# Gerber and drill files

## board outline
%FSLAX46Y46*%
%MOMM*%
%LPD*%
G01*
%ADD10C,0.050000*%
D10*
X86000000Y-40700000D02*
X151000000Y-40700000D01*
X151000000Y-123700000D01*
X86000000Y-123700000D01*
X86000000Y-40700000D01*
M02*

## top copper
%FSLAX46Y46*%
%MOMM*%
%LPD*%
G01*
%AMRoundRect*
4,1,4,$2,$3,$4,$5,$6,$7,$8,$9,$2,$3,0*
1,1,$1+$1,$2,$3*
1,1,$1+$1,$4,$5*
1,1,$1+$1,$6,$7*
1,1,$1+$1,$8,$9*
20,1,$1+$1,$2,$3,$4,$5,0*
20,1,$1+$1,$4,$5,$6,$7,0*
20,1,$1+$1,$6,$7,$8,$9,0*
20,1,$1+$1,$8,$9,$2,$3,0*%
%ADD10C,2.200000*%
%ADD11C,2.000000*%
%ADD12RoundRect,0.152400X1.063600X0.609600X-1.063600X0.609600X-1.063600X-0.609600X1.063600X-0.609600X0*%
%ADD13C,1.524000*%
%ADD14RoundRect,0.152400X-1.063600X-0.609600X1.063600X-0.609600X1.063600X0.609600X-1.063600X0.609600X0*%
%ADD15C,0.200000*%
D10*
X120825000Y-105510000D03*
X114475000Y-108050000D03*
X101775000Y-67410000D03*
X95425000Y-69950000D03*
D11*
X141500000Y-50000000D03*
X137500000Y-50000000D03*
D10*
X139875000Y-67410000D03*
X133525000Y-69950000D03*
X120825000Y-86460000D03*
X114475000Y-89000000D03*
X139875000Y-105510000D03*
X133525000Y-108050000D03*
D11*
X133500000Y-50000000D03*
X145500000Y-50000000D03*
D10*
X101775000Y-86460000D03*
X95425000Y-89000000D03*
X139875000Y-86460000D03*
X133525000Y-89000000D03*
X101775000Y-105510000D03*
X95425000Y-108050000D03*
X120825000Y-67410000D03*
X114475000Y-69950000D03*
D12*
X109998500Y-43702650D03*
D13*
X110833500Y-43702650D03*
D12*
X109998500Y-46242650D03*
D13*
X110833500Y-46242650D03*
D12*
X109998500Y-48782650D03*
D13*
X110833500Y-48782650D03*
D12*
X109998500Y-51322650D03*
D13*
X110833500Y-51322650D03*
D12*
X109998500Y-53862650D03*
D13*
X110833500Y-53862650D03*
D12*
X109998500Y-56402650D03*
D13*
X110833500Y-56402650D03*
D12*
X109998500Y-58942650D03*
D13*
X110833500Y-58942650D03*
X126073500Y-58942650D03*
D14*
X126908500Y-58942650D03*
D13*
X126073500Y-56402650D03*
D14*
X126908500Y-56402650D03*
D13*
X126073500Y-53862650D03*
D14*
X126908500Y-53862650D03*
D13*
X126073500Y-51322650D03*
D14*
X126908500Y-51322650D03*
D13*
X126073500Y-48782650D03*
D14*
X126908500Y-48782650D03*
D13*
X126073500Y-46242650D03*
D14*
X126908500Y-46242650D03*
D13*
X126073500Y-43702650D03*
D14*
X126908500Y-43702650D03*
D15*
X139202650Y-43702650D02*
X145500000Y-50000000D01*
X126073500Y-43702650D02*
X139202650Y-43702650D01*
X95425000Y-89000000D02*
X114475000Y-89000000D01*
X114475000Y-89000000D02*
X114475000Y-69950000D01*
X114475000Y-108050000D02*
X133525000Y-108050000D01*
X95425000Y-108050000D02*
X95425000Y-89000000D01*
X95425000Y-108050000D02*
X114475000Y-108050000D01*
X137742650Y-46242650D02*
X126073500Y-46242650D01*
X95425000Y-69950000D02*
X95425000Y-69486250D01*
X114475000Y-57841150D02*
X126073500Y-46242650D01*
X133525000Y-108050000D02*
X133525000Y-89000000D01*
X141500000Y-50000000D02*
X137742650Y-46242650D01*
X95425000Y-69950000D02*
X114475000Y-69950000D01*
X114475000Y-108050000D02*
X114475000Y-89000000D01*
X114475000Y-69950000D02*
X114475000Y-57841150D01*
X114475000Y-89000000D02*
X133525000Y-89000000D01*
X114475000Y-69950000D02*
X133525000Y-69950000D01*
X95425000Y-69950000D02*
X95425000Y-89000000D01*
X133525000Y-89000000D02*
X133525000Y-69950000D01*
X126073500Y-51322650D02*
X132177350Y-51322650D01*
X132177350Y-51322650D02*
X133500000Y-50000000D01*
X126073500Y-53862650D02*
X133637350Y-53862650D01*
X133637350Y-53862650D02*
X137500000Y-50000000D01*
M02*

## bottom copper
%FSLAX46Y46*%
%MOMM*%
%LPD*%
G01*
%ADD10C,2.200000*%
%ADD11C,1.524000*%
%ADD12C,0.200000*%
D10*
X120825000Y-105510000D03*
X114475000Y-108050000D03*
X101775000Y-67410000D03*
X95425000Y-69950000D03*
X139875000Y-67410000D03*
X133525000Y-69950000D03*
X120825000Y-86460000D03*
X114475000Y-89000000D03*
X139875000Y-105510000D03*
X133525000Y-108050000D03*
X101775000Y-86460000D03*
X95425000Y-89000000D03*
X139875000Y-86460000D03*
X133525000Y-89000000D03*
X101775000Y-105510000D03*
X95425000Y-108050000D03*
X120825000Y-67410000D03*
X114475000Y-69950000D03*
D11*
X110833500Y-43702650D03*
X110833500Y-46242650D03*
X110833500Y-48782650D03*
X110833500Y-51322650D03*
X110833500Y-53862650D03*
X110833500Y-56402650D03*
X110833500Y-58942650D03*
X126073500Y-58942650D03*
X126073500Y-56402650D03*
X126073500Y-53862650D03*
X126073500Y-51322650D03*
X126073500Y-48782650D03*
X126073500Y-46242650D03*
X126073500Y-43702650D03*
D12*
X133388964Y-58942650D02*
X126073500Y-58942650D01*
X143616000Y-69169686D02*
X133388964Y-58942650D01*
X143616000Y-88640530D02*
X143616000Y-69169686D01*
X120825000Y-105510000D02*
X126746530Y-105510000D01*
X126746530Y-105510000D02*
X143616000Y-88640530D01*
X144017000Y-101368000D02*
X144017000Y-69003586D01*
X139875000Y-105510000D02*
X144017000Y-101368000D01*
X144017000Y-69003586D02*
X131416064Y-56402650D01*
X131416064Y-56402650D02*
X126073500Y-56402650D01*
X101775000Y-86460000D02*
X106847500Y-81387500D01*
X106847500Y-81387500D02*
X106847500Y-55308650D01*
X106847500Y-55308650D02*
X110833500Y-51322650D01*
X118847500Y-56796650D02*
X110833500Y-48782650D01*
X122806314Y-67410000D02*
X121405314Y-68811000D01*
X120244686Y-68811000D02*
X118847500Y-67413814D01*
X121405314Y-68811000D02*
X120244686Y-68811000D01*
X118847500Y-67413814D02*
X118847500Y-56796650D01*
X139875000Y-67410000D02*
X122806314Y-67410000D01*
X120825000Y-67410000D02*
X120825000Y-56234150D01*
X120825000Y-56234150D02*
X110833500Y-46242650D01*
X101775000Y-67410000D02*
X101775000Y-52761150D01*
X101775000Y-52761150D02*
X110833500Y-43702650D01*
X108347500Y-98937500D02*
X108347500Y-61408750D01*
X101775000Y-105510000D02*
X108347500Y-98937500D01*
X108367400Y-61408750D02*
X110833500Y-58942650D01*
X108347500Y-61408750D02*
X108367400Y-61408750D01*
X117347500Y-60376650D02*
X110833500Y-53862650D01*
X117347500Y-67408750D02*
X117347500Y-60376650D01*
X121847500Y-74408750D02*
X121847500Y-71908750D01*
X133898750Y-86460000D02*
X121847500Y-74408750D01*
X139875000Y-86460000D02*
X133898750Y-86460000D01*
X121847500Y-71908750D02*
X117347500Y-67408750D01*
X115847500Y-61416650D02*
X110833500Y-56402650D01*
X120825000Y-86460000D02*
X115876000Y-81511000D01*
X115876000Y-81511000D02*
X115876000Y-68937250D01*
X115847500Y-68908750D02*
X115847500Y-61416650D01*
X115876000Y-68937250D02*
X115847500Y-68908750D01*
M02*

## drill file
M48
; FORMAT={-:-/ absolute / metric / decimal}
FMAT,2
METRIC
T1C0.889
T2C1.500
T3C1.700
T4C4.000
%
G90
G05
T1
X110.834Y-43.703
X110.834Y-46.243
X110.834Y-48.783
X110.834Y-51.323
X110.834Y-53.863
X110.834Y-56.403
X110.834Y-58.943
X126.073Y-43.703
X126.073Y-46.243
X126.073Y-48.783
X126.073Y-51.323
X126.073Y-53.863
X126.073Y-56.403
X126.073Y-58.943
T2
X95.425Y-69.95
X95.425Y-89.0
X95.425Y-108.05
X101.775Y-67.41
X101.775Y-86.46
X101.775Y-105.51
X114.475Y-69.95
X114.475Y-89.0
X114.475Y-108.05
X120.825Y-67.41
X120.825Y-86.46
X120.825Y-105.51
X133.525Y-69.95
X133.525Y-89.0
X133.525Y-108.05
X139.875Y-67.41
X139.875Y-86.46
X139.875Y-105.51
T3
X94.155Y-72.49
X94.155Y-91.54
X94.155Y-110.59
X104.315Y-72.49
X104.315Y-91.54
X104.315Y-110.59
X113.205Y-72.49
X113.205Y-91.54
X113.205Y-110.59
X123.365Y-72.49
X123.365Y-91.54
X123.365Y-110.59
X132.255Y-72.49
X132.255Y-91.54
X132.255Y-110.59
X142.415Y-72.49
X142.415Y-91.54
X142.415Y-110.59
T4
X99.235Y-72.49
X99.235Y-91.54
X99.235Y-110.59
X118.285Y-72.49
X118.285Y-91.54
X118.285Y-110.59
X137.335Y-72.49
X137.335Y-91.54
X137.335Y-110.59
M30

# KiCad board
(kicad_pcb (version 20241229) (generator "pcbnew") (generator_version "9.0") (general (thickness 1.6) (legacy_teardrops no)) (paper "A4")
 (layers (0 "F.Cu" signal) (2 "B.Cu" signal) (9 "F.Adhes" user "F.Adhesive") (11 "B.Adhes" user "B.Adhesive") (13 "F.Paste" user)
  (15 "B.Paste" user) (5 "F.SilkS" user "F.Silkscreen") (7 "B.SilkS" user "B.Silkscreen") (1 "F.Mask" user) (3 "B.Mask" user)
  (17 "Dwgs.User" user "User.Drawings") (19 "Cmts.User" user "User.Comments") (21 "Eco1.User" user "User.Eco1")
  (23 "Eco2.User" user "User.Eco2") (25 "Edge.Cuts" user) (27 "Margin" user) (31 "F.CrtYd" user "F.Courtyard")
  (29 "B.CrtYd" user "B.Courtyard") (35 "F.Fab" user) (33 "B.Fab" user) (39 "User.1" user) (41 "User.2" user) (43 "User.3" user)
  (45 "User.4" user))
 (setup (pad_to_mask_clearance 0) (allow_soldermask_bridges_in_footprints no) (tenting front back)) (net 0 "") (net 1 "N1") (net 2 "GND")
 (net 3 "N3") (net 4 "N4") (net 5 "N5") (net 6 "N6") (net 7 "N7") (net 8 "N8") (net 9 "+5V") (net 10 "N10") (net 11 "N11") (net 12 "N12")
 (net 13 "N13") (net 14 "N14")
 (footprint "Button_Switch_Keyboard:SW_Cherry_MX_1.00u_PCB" (layer "F.Cu") (at 120.825 105.51)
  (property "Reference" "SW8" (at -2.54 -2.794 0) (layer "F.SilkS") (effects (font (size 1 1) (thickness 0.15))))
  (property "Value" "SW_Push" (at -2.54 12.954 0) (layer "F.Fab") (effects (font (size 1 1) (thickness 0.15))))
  (pad "" np_thru_hole circle (at -7.62 5.08) (size 1.7 1.7) (drill 1.7) (layers "*.Cu" "*.Mask"))
  (pad "" np_thru_hole circle (at -2.54 5.08) (size 4 4) (drill 4) (layers "*.Cu" "*.Mask"))
  (pad "" np_thru_hole circle (at 2.54 5.08) (size 1.7 1.7) (drill 1.7) (layers "*.Cu" "*.Mask"))
  (pad "1" thru_hole circle (at 0 0) (size 2.2 2.2) (drill 1.5) (layers "*.Cu" "*.Mask") (remove_unused_layers no) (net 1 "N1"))
  (pad "2" thru_hole circle (at -6.35 2.54) (size 2.2 2.2) (drill 1.5) (layers "*.Cu" "*.Mask") (remove_unused_layers no) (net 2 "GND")))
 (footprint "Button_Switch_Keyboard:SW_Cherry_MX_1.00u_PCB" (layer "F.Cu") (at 101.775 67.41)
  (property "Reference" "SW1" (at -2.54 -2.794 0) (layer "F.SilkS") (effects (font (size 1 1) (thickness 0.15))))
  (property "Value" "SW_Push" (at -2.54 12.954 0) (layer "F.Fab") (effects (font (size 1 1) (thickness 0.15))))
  (pad "" np_thru_hole circle (at -7.62 5.08) (size 1.7 1.7) (drill 1.7) (layers "*.Cu" "*.Mask"))
  (pad "" np_thru_hole circle (at -2.54 5.08) (size 4 4) (drill 4) (layers "*.Cu" "*.Mask"))
  (pad "" np_thru_hole circle (at 2.54 5.08) (size 1.7 1.7) (drill 1.7) (layers "*.Cu" "*.Mask"))
  (pad "1" thru_hole circle (at 0 0) (size 2.2 2.2) (drill 1.5) (layers "*.Cu" "*.Mask") (remove_unused_layers no) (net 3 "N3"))
  (pad "2" thru_hole circle (at -6.35 2.54) (size 2.2 2.2) (drill 1.5) (layers "*.Cu" "*.Mask") (remove_unused_layers no) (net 2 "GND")))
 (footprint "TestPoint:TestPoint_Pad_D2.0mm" (layer "F.Cu") (at 141.5 50)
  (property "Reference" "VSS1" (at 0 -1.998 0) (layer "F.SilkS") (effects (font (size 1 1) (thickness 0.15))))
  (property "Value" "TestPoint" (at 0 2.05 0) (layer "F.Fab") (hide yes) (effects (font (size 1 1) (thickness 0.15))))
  (pad "1" smd circle (at 0 0) (size 2 2) (layers "F.Cu" "F.Mask") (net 2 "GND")))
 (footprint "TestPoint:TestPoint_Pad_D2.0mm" (layer "F.Cu") (at 137.5 50)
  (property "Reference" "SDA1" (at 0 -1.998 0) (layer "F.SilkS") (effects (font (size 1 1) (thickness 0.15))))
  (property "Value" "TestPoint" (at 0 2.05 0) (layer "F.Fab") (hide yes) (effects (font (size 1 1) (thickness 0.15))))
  (pad "1" smd circle (at 0 0) (size 2 2) (layers "F.Cu" "F.Mask") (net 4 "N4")))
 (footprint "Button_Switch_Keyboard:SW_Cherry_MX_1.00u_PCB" (layer "F.Cu") (at 139.875 67.41)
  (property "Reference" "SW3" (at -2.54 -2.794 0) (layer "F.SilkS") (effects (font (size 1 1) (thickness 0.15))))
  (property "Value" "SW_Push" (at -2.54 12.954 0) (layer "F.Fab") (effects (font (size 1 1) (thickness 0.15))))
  (pad "" np_thru_hole circle (at -7.62 5.08) (size 1.7 1.7) (drill 1.7) (layers "*.Cu" "*.Mask"))
  (pad "" np_thru_hole circle (at -2.54 5.08) (size 4 4) (drill 4) (layers "*.Cu" "*.Mask"))
  (pad "" np_thru_hole circle (at 2.54 5.08) (size 1.7 1.7) (drill 1.7) (layers "*.Cu" "*.Mask"))
  (pad "1" thru_hole circle (at 0 0) (size 2.2 2.2) (drill 1.5) (layers "*.Cu" "*.Mask") (remove_unused_layers no) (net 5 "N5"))
  (pad "2" thru_hole circle (at -6.35 2.54) (size 2.2 2.2) (drill 1.5) (layers "*.Cu" "*.Mask") (remove_unused_layers no) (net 2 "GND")))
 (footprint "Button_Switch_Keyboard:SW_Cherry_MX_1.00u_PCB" (layer "F.Cu") (at 120.825 86.46)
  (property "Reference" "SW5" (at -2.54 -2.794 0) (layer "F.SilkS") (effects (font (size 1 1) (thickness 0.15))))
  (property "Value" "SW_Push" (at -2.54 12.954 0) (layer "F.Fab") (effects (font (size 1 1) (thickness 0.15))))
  (pad "" np_thru_hole circle (at -7.62 5.08) (size 1.7 1.7) (drill 1.7) (layers "*.Cu" "*.Mask"))
  (pad "" np_thru_hole circle (at -2.54 5.08) (size 4 4) (drill 4) (layers "*.Cu" "*.Mask"))
  (pad "" np_thru_hole circle (at 2.54 5.08) (size 1.7 1.7) (drill 1.7) (layers "*.Cu" "*.Mask"))
  (pad "1" thru_hole circle (at 0 0) (size 2.2 2.2) (drill 1.5) (layers "*.Cu" "*.Mask") (remove_unused_layers no) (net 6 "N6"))
  (pad "2" thru_hole circle (at -6.35 2.54) (size 2.2 2.2) (drill 1.5) (layers "*.Cu" "*.Mask") (remove_unused_layers no) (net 2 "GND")))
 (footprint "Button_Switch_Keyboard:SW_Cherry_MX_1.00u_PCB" (layer "F.Cu") (at 139.875 105.51)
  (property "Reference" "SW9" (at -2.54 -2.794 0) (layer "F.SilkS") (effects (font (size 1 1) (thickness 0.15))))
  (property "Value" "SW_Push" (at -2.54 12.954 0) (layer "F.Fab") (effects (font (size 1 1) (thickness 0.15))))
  (pad "" np_thru_hole circle (at -7.62 5.08) (size 1.7 1.7) (drill 1.7) (layers "*.Cu" "*.Mask"))
  (pad "" np_thru_hole circle (at -2.54 5.08) (size 4 4) (drill 4) (layers "*.Cu" "*.Mask"))
  (pad "" np_thru_hole circle (at 2.54 5.08) (size 1.7 1.7) (drill 1.7) (layers "*.Cu" "*.Mask"))
  (pad "1" thru_hole circle (at 0 0) (size 2.2 2.2) (drill 1.5) (layers "*.Cu" "*.Mask") (remove_unused_layers no) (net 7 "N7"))
  (pad "2" thru_hole circle (at -6.35 2.54) (size 2.2 2.2) (drill 1.5) (layers "*.Cu" "*.Mask") (remove_unused_layers no) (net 2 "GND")))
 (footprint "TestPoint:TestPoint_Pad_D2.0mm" (layer "F.Cu") (at 133.5 50)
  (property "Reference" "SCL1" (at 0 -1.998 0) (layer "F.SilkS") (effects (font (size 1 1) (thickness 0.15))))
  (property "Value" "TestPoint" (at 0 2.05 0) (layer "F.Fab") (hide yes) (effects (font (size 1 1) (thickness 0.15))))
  (pad "1" smd circle (at 0 0) (size 2 2) (layers "F.Cu" "F.Mask") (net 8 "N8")))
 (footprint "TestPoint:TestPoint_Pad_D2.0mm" (layer "F.Cu") (at 145.5 50)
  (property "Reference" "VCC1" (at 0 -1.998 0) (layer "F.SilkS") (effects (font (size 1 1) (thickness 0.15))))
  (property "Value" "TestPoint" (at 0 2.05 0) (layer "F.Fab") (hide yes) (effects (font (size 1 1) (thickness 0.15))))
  (pad "1" smd circle (at 0 0) (size 2 2) (layers "F.Cu" "F.Mask") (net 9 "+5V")))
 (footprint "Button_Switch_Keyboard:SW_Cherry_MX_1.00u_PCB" (layer "F.Cu") (at 101.775 86.46)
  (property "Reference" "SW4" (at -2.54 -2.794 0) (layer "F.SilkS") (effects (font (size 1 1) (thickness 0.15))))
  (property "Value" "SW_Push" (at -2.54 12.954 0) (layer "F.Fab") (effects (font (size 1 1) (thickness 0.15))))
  (pad "" np_thru_hole circle (at -7.62 5.08) (size 1.7 1.7) (drill 1.7) (layers "*.Cu" "*.Mask"))
  (pad "" np_thru_hole circle (at -2.54 5.08) (size 4 4) (drill 4) (layers "*.Cu" "*.Mask"))
  (pad "" np_thru_hole circle (at 2.54 5.08) (size 1.7 1.7) (drill 1.7) (layers "*.Cu" "*.Mask"))
  (pad "1" thru_hole circle (at 0 0) (size 2.2 2.2) (drill 1.5) (layers "*.Cu" "*.Mask") (remove_unused_layers no) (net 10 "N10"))
  (pad "2" thru_hole circle (at -6.35 2.54) (size 2.2 2.2) (drill 1.5) (layers "*.Cu" "*.Mask") (remove_unused_layers no) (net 2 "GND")))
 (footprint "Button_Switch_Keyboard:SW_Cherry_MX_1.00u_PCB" (layer "F.Cu") (at 139.875 86.46)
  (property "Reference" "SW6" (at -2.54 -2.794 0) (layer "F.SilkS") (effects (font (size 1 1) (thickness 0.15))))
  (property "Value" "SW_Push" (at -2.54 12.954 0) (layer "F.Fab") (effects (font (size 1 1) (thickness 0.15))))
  (pad "" np_thru_hole circle (at -7.62 5.08) (size 1.7 1.7) (drill 1.7) (layers "*.Cu" "*.Mask"))
  (pad "" np_thru_hole circle (at -2.54 5.08) (size 4 4) (drill 4) (layers "*.Cu" "*.Mask"))
  (pad "" np_thru_hole circle (at 2.54 5.08) (size 1.7 1.7) (drill 1.7) (layers "*.Cu" "*.Mask"))
  (pad "1" thru_hole circle (at 0 0) (size 2.2 2.2) (drill 1.5) (layers "*.Cu" "*.Mask") (remove_unused_layers no) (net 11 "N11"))
  (pad "2" thru_hole circle (at -6.35 2.54) (size 2.2 2.2) (drill 1.5) (layers "*.Cu" "*.Mask") (remove_unused_layers no) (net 2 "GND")))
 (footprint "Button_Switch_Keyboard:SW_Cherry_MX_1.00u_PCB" (layer "F.Cu") (at 101.775 105.51)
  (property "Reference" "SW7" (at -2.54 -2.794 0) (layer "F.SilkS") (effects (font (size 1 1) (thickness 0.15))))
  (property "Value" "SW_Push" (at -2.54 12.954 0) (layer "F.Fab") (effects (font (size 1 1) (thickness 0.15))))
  (pad "" np_thru_hole circle (at -7.62 5.08) (size 1.7 1.7) (drill 1.7) (layers "*.Cu" "*.Mask"))
  (pad "" np_thru_hole circle (at -2.54 5.08) (size 4 4) (drill 4) (layers "*.Cu" "*.Mask"))
  (pad "" np_thru_hole circle (at 2.54 5.08) (size 1.7 1.7) (drill 1.7) (layers "*.Cu" "*.Mask"))
  (pad "1" thru_hole circle (at 0 0) (size 2.2 2.2) (drill 1.5) (layers "*.Cu" "*.Mask") (remove_unused_layers no) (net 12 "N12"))
  (pad "2" thru_hole circle (at -6.35 2.54) (size 2.2 2.2) (drill 1.5) (layers "*.Cu" "*.Mask") (remove_unused_layers no) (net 2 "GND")))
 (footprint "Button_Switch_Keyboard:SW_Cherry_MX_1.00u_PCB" (layer "F.Cu") (at 120.825 67.41)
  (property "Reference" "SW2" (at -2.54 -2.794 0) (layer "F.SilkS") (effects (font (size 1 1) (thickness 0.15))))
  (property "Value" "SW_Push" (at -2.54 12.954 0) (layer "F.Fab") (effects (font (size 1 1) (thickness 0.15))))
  (pad "" np_thru_hole circle (at -7.62 5.08) (size 1.7 1.7) (drill 1.7) (layers "*.Cu" "*.Mask"))
  (pad "" np_thru_hole circle (at -2.54 5.08) (size 4 4) (drill 4) (layers "*.Cu" "*.Mask"))
  (pad "" np_thru_hole circle (at 2.54 5.08) (size 1.7 1.7) (drill 1.7) (layers "*.Cu" "*.Mask"))
  (pad "1" thru_hole circle (at 0 0) (size 2.2 2.2) (drill 1.5) (layers "*.Cu" "*.Mask") (remove_unused_layers no) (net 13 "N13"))
  (pad "2" thru_hole circle (at -6.35 2.54) (size 2.2 2.2) (drill 1.5) (layers "*.Cu" "*.Mask") (remove_unused_layers no) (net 2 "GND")))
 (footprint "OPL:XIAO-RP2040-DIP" (layer "F.Cu") (at 118.4535 51.32265)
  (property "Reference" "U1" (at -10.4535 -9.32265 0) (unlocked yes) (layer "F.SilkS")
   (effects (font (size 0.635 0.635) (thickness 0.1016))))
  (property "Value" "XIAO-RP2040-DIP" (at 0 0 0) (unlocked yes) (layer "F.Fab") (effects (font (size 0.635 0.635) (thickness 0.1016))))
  (pad "1" smd roundrect (at -8.455 -7.62 180) (size 2.432 1.524) (layers "F.Cu" "F.Mask") (roundrect_rratio 0.1) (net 3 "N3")
   (thermal_bridge_angle 45))
  (pad "1" thru_hole circle (at -7.62 -7.62 180) (size 1.524 1.524) (drill 0.889) (layers "*.Cu" "*.Mask") (remove_unused_layers no)
   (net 3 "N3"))
  (pad "2" smd roundrect (at -8.455 -5.08 180) (size 2.432 1.524) (layers "F.Cu" "F.Mask") (roundrect_rratio 0.1) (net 13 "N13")
   (thermal_bridge_angle 45))
  (pad "2" thru_hole circle (at -7.62 -5.08 180) (size 1.524 1.524) (drill 0.889) (layers "*.Cu" "*.Mask") (remove_unused_layers no)
   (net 13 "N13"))
  (pad "3" smd roundrect (at -8.455 -2.54 180) (size 2.432 1.524) (layers "F.Cu" "F.Mask") (roundrect_rratio 0.1) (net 5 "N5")
   (thermal_bridge_angle 45))
  (pad "3" thru_hole circle (at -7.62 -2.54 180) (size 1.524 1.524) (drill 0.889) (layers "*.Cu" "*.Mask") (remove_unused_layers no)
   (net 5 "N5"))
  (pad "4" smd roundrect (at -8.455 0 180) (size 2.432 1.524) (layers "F.Cu" "F.Mask") (roundrect_rratio 0.1) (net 10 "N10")
   (thermal_bridge_angle 45))
  (pad "4" thru_hole circle (at -7.62 0 180) (size 1.524 1.524) (drill 0.889) (layers "*.Cu" "*.Mask") (remove_unused_layers no)
   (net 10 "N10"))
  (pad "5" smd roundrect (at -8.455 2.54 180) (size 2.432 1.524) (layers "F.Cu" "F.Mask") (roundrect_rratio 0.1) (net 11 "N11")
   (thermal_bridge_angle 45))
  (pad "5" thru_hole circle (at -7.62 2.54 180) (size 1.524 1.524) (drill 0.889) (layers "*.Cu" "*.Mask") (remove_unused_layers no)
   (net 11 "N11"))
  (pad "6" smd roundrect (at -8.455 5.08 180) (size 2.432 1.524) (layers "F.Cu" "F.Mask") (roundrect_rratio 0.1) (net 6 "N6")
   (thermal_bridge_angle 45))
  (pad "6" thru_hole circle (at -7.62 5.08 180) (size 1.524 1.524) (drill 0.889) (layers "*.Cu" "*.Mask") (remove_unused_layers no)
   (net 6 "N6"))
  (pad "7" smd roundrect (at -8.455 7.62 180) (size 2.432 1.524) (layers "F.Cu" "F.Mask") (roundrect_rratio 0.1) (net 12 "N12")
   (thermal_bridge_angle 45))
  (pad "7" thru_hole circle (at -7.62 7.62 180) (size 1.524 1.524) (drill 0.889) (layers "*.Cu" "*.Mask") (remove_unused_layers no)
   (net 12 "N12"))
  (pad "8" thru_hole circle (at 7.62 7.62) (size 1.524 1.524) (drill 0.889) (layers "*.Cu" "*.Mask") (remove_unused_layers no) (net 1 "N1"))
  (pad "8" smd roundrect (at 8.455 7.62) (size 2.432 1.524) (layers "F.Cu" "F.Mask") (roundrect_rratio 0.1) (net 1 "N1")
   (thermal_bridge_angle 45))
  (pad "9" thru_hole circle (at 7.62 5.08) (size 1.524 1.524) (drill 0.889) (layers "*.Cu" "*.Mask") (remove_unused_layers no) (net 7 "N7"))
  (pad "9" smd roundrect (at 8.455 5.08) (size 2.432 1.524) (layers "F.Cu" "F.Mask") (roundrect_rratio 0.1) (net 7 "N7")
   (thermal_bridge_angle 45))
  (pad "10" thru_hole circle (at 7.62 2.54) (size 1.524 1.524) (drill 0.889) (layers "*.Cu" "*.Mask") (remove_unused_layers no) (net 4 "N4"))
  (pad "10" smd roundrect (at 8.455 2.54) (size 2.432 1.524) (layers "F.Cu" "F.Mask") (roundrect_rratio 0.1) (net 4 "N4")
   (thermal_bridge_angle 45))
  (pad "11" thru_hole circle (at 7.62 0) (size 1.524 1.524) (drill 0.889) (layers "*.Cu" "*.Mask") (remove_unused_layers no) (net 8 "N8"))
  (pad "11" smd roundrect (at 8.455 0) (size 2.432 1.524) (layers "F.Cu" "F.Mask") (roundrect_rratio 0.1) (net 8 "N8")
   (thermal_bridge_angle 45))
  (pad "12" thru_hole circle (at 7.62 -2.54) (size 1.524 1.524) (drill 0.889) (layers "*.Cu" "*.Mask") (remove_unused_layers no)
   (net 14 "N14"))
  (pad "12" smd roundrect (at 8.455 -2.54) (size 2.432 1.524) (layers "F.Cu" "F.Mask") (roundrect_rratio 0.1) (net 14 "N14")
   (thermal_bridge_angle 45))
  (pad "13" thru_hole circle (at 7.62 -5.08) (size 1.524 1.524) (drill 0.889) (layers "*.Cu" "*.Mask") (remove_unused_layers no)
   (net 2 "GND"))
  (pad "13" smd roundrect (at 8.455 -5.08) (size 2.432 1.524) (layers "F.Cu" "F.Mask") (roundrect_rratio 0.1) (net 2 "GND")
   (thermal_bridge_angle 45))
  (pad "14" thru_hole circle (at 7.62 -7.62) (size 1.524 1.524) (drill 0.889) (layers "*.Cu" "*.Mask") (remove_unused_layers no)
   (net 9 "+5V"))
  (pad "14" smd roundrect (at 8.455 -7.62) (size 2.432 1.524) (layers "F.Cu" "F.Mask") (roundrect_rratio 0.1) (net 9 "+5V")
   (thermal_bridge_angle 45)))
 (gr_rect (start 86 40.7) (end 151 123.7) (stroke (width 0.05) (type default)) (fill no) (layer "Edge.Cuts"))
 (segment (start 139.20265 43.70265) (end 145.5 50) (width 0.2) (layer "F.Cu") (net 9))
 (segment (start 126.0735 43.70265) (end 139.20265 43.70265) (width 0.2) (layer "F.Cu") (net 9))
 (segment (start 95.425 89) (end 114.475 89) (width 0.2) (layer "F.Cu") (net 2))
 (segment (start 114.475 89) (end 114.475 69.95) (width 0.2) (layer "F.Cu") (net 2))
 (segment (start 114.475 108.05) (end 133.525 108.05) (width 0.2) (layer "F.Cu") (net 2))
 (segment (start 95.425 108.05) (end 95.425 89) (width 0.2) (layer "F.Cu") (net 2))
 (segment (start 95.425 108.05) (end 114.475 108.05) (width 0.2) (layer "F.Cu") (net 2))
 (segment (start 137.74265 46.24265) (end 126.0735 46.24265) (width 0.2) (layer "F.Cu") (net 2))
 (segment (start 95.425 69.95) (end 95.425 69.48625) (width 0.2) (layer "F.Cu") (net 2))
 (segment (start 114.475 57.84115) (end 126.0735 46.24265) (width 0.2) (layer "F.Cu") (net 2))
 (segment (start 133.525 108.05) (end 133.525 89) (width 0.2) (layer "F.Cu") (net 2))
 (segment (start 141.5 50) (end 137.74265 46.24265) (width 0.2) (layer "F.Cu") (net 2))
 (segment (start 95.425 69.95) (end 114.475 69.95) (width 0.2) (layer "F.Cu") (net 2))
 (segment (start 114.475 108.05) (end 114.475 89) (width 0.2) (layer "F.Cu") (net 2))
 (segment (start 114.475 69.95) (end 114.475 57.84115) (width 0.2) (layer "F.Cu") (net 2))
 (segment (start 114.475 89) (end 133.525 89) (width 0.2) (layer "F.Cu") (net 2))
 (segment (start 114.475 69.95) (end 133.525 69.95) (width 0.2) (layer "F.Cu") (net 2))
 (segment (start 95.425 69.95) (end 95.425 89) (width 0.2) (layer "F.Cu") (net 2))
 (segment (start 133.525 89) (end 133.525 69.95) (width 0.2) (layer "F.Cu") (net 2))
 (segment (start 133.388964 58.94265) (end 126.0735 58.94265) (width 0.2) (layer "B.Cu") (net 1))
 (segment (start 143.616 69.169686) (end 133.388964 58.94265) (width 0.2) (layer "B.Cu") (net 1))
 (segment (start 143.616 88.64053) (end 143.616 69.169686) (width 0.2) (layer "B.Cu") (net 1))
 (segment (start 120.825 105.51) (end 126.74653 105.51) (width 0.2) (layer "B.Cu") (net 1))
 (segment (start 126.74653 105.51) (end 143.616 88.64053) (width 0.2) (layer "B.Cu") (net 1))
 (segment (start 144.017 101.368) (end 144.017 69.003586) (width 0.2) (layer "B.Cu") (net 7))
 (segment (start 139.875 105.51) (end 144.017 101.368) (width 0.2) (layer "B.Cu") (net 7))
 (segment (start 144.017 69.003586) (end 131.416064 56.40265) (width 0.2) (layer "B.Cu") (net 7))
 (segment (start 131.416064 56.40265) (end 126.0735 56.40265) (width 0.2) (layer "B.Cu") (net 7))
 (segment (start 101.775 86.46) (end 106.8475 81.3875) (width 0.2) (layer "B.Cu") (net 10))
 (segment (start 106.8475 81.3875) (end 106.8475 55.30865) (width 0.2) (layer "B.Cu") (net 10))
 (segment (start 106.8475 55.30865) (end 110.8335 51.32265) (width 0.2) (layer "B.Cu") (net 10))
 (segment (start 118.8475 56.79665) (end 110.8335 48.78265) (width 0.2) (layer "B.Cu") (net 5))
 (segment (start 122.806314 67.41) (end 121.405314 68.811) (width 0.2) (layer "B.Cu") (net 5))
 (segment (start 120.244686 68.811) (end 118.8475 67.413814) (width 0.2) (layer "B.Cu") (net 5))
 (segment (start 121.405314 68.811) (end 120.244686 68.811) (width 0.2) (layer "B.Cu") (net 5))
 (segment (start 118.8475 67.413814) (end 118.8475 56.79665) (width 0.2) (layer "B.Cu") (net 5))
 (segment (start 139.875 67.41) (end 122.806314 67.41) (width 0.2) (layer "B.Cu") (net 5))
 (segment (start 120.825 67.41) (end 120.825 56.23415) (width 0.2) (layer "B.Cu") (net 13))
 (segment (start 120.825 56.23415) (end 110.8335 46.24265) (width 0.2) (layer "B.Cu") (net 13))
 (segment (start 101.775 67.41) (end 101.775 52.76115) (width 0.2) (layer "B.Cu") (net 3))
 (segment (start 101.775 52.76115) (end 110.8335 43.70265) (width 0.2) (layer "B.Cu") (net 3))
 (segment (start 108.3475 98.9375) (end 108.3475 61.40875) (width 0.2) (layer "B.Cu") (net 12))
 (segment (start 101.775 105.51) (end 108.3475 98.9375) (width 0.2) (layer "B.Cu") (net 12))
 (segment (start 108.3674 61.40875) (end 110.8335 58.94265) (width 0.2) (layer "B.Cu") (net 12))
 (segment (start 108.3475 61.40875) (end 108.3674 61.40875) (width 0.2) (layer "B.Cu") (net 12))
 (segment (start 117.3475 60.37665) (end 110.8335 53.86265) (width 0.2) (layer "B.Cu") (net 11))
 (segment (start 117.3475 67.40875) (end 117.3475 60.37665) (width 0.2) (layer "B.Cu") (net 11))
 (segment (start 121.8475 74.40875) (end 121.8475 71.90875) (width 0.2) (layer "B.Cu") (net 11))
 (segment (start 133.89875 86.46) (end 121.8475 74.40875) (width 0.2) (layer "B.Cu") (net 11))
 (segment (start 139.875 86.46) (end 133.89875 86.46) (width 0.2) (layer "B.Cu") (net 11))
 (segment (start 121.8475 71.90875) (end 117.3475 67.40875) (width 0.2) (layer "B.Cu") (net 11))
 (segment (start 115.8475 61.41665) (end 110.8335 56.40265) (width 0.2) (layer "B.Cu") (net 6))
 (segment (start 120.825 86.46) (end 115.876 81.511) (width 0.2) (layer "B.Cu") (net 6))
 (segment (start 115.876 81.511) (end 115.876 68.93725) (width 0.2) (layer "B.Cu") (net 6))
 (segment (start 115.8475 68.90875) (end 115.8475 61.41665) (width 0.2) (layer "B.Cu") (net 6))
 (segment (start 115.876 68.93725) (end 115.8475 68.90875) (width 0.2) (layer "B.Cu") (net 6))
 (segment (start 126.0735 51.32265) (end 132.17735 51.32265) (width 0.2) (layer "F.Cu") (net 8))
 (segment (start 132.17735 51.32265) (end 133.5 50) (width 0.2) (layer "F.Cu") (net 8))
 (segment (start 126.0735 53.86265) (end 133.63735 53.86265) (width 0.2) (layer "F.Cu") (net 4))
 (segment (start 133.63735 53.86265) (end 137.5 50) (width 0.2) (layer "F.Cu") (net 4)))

